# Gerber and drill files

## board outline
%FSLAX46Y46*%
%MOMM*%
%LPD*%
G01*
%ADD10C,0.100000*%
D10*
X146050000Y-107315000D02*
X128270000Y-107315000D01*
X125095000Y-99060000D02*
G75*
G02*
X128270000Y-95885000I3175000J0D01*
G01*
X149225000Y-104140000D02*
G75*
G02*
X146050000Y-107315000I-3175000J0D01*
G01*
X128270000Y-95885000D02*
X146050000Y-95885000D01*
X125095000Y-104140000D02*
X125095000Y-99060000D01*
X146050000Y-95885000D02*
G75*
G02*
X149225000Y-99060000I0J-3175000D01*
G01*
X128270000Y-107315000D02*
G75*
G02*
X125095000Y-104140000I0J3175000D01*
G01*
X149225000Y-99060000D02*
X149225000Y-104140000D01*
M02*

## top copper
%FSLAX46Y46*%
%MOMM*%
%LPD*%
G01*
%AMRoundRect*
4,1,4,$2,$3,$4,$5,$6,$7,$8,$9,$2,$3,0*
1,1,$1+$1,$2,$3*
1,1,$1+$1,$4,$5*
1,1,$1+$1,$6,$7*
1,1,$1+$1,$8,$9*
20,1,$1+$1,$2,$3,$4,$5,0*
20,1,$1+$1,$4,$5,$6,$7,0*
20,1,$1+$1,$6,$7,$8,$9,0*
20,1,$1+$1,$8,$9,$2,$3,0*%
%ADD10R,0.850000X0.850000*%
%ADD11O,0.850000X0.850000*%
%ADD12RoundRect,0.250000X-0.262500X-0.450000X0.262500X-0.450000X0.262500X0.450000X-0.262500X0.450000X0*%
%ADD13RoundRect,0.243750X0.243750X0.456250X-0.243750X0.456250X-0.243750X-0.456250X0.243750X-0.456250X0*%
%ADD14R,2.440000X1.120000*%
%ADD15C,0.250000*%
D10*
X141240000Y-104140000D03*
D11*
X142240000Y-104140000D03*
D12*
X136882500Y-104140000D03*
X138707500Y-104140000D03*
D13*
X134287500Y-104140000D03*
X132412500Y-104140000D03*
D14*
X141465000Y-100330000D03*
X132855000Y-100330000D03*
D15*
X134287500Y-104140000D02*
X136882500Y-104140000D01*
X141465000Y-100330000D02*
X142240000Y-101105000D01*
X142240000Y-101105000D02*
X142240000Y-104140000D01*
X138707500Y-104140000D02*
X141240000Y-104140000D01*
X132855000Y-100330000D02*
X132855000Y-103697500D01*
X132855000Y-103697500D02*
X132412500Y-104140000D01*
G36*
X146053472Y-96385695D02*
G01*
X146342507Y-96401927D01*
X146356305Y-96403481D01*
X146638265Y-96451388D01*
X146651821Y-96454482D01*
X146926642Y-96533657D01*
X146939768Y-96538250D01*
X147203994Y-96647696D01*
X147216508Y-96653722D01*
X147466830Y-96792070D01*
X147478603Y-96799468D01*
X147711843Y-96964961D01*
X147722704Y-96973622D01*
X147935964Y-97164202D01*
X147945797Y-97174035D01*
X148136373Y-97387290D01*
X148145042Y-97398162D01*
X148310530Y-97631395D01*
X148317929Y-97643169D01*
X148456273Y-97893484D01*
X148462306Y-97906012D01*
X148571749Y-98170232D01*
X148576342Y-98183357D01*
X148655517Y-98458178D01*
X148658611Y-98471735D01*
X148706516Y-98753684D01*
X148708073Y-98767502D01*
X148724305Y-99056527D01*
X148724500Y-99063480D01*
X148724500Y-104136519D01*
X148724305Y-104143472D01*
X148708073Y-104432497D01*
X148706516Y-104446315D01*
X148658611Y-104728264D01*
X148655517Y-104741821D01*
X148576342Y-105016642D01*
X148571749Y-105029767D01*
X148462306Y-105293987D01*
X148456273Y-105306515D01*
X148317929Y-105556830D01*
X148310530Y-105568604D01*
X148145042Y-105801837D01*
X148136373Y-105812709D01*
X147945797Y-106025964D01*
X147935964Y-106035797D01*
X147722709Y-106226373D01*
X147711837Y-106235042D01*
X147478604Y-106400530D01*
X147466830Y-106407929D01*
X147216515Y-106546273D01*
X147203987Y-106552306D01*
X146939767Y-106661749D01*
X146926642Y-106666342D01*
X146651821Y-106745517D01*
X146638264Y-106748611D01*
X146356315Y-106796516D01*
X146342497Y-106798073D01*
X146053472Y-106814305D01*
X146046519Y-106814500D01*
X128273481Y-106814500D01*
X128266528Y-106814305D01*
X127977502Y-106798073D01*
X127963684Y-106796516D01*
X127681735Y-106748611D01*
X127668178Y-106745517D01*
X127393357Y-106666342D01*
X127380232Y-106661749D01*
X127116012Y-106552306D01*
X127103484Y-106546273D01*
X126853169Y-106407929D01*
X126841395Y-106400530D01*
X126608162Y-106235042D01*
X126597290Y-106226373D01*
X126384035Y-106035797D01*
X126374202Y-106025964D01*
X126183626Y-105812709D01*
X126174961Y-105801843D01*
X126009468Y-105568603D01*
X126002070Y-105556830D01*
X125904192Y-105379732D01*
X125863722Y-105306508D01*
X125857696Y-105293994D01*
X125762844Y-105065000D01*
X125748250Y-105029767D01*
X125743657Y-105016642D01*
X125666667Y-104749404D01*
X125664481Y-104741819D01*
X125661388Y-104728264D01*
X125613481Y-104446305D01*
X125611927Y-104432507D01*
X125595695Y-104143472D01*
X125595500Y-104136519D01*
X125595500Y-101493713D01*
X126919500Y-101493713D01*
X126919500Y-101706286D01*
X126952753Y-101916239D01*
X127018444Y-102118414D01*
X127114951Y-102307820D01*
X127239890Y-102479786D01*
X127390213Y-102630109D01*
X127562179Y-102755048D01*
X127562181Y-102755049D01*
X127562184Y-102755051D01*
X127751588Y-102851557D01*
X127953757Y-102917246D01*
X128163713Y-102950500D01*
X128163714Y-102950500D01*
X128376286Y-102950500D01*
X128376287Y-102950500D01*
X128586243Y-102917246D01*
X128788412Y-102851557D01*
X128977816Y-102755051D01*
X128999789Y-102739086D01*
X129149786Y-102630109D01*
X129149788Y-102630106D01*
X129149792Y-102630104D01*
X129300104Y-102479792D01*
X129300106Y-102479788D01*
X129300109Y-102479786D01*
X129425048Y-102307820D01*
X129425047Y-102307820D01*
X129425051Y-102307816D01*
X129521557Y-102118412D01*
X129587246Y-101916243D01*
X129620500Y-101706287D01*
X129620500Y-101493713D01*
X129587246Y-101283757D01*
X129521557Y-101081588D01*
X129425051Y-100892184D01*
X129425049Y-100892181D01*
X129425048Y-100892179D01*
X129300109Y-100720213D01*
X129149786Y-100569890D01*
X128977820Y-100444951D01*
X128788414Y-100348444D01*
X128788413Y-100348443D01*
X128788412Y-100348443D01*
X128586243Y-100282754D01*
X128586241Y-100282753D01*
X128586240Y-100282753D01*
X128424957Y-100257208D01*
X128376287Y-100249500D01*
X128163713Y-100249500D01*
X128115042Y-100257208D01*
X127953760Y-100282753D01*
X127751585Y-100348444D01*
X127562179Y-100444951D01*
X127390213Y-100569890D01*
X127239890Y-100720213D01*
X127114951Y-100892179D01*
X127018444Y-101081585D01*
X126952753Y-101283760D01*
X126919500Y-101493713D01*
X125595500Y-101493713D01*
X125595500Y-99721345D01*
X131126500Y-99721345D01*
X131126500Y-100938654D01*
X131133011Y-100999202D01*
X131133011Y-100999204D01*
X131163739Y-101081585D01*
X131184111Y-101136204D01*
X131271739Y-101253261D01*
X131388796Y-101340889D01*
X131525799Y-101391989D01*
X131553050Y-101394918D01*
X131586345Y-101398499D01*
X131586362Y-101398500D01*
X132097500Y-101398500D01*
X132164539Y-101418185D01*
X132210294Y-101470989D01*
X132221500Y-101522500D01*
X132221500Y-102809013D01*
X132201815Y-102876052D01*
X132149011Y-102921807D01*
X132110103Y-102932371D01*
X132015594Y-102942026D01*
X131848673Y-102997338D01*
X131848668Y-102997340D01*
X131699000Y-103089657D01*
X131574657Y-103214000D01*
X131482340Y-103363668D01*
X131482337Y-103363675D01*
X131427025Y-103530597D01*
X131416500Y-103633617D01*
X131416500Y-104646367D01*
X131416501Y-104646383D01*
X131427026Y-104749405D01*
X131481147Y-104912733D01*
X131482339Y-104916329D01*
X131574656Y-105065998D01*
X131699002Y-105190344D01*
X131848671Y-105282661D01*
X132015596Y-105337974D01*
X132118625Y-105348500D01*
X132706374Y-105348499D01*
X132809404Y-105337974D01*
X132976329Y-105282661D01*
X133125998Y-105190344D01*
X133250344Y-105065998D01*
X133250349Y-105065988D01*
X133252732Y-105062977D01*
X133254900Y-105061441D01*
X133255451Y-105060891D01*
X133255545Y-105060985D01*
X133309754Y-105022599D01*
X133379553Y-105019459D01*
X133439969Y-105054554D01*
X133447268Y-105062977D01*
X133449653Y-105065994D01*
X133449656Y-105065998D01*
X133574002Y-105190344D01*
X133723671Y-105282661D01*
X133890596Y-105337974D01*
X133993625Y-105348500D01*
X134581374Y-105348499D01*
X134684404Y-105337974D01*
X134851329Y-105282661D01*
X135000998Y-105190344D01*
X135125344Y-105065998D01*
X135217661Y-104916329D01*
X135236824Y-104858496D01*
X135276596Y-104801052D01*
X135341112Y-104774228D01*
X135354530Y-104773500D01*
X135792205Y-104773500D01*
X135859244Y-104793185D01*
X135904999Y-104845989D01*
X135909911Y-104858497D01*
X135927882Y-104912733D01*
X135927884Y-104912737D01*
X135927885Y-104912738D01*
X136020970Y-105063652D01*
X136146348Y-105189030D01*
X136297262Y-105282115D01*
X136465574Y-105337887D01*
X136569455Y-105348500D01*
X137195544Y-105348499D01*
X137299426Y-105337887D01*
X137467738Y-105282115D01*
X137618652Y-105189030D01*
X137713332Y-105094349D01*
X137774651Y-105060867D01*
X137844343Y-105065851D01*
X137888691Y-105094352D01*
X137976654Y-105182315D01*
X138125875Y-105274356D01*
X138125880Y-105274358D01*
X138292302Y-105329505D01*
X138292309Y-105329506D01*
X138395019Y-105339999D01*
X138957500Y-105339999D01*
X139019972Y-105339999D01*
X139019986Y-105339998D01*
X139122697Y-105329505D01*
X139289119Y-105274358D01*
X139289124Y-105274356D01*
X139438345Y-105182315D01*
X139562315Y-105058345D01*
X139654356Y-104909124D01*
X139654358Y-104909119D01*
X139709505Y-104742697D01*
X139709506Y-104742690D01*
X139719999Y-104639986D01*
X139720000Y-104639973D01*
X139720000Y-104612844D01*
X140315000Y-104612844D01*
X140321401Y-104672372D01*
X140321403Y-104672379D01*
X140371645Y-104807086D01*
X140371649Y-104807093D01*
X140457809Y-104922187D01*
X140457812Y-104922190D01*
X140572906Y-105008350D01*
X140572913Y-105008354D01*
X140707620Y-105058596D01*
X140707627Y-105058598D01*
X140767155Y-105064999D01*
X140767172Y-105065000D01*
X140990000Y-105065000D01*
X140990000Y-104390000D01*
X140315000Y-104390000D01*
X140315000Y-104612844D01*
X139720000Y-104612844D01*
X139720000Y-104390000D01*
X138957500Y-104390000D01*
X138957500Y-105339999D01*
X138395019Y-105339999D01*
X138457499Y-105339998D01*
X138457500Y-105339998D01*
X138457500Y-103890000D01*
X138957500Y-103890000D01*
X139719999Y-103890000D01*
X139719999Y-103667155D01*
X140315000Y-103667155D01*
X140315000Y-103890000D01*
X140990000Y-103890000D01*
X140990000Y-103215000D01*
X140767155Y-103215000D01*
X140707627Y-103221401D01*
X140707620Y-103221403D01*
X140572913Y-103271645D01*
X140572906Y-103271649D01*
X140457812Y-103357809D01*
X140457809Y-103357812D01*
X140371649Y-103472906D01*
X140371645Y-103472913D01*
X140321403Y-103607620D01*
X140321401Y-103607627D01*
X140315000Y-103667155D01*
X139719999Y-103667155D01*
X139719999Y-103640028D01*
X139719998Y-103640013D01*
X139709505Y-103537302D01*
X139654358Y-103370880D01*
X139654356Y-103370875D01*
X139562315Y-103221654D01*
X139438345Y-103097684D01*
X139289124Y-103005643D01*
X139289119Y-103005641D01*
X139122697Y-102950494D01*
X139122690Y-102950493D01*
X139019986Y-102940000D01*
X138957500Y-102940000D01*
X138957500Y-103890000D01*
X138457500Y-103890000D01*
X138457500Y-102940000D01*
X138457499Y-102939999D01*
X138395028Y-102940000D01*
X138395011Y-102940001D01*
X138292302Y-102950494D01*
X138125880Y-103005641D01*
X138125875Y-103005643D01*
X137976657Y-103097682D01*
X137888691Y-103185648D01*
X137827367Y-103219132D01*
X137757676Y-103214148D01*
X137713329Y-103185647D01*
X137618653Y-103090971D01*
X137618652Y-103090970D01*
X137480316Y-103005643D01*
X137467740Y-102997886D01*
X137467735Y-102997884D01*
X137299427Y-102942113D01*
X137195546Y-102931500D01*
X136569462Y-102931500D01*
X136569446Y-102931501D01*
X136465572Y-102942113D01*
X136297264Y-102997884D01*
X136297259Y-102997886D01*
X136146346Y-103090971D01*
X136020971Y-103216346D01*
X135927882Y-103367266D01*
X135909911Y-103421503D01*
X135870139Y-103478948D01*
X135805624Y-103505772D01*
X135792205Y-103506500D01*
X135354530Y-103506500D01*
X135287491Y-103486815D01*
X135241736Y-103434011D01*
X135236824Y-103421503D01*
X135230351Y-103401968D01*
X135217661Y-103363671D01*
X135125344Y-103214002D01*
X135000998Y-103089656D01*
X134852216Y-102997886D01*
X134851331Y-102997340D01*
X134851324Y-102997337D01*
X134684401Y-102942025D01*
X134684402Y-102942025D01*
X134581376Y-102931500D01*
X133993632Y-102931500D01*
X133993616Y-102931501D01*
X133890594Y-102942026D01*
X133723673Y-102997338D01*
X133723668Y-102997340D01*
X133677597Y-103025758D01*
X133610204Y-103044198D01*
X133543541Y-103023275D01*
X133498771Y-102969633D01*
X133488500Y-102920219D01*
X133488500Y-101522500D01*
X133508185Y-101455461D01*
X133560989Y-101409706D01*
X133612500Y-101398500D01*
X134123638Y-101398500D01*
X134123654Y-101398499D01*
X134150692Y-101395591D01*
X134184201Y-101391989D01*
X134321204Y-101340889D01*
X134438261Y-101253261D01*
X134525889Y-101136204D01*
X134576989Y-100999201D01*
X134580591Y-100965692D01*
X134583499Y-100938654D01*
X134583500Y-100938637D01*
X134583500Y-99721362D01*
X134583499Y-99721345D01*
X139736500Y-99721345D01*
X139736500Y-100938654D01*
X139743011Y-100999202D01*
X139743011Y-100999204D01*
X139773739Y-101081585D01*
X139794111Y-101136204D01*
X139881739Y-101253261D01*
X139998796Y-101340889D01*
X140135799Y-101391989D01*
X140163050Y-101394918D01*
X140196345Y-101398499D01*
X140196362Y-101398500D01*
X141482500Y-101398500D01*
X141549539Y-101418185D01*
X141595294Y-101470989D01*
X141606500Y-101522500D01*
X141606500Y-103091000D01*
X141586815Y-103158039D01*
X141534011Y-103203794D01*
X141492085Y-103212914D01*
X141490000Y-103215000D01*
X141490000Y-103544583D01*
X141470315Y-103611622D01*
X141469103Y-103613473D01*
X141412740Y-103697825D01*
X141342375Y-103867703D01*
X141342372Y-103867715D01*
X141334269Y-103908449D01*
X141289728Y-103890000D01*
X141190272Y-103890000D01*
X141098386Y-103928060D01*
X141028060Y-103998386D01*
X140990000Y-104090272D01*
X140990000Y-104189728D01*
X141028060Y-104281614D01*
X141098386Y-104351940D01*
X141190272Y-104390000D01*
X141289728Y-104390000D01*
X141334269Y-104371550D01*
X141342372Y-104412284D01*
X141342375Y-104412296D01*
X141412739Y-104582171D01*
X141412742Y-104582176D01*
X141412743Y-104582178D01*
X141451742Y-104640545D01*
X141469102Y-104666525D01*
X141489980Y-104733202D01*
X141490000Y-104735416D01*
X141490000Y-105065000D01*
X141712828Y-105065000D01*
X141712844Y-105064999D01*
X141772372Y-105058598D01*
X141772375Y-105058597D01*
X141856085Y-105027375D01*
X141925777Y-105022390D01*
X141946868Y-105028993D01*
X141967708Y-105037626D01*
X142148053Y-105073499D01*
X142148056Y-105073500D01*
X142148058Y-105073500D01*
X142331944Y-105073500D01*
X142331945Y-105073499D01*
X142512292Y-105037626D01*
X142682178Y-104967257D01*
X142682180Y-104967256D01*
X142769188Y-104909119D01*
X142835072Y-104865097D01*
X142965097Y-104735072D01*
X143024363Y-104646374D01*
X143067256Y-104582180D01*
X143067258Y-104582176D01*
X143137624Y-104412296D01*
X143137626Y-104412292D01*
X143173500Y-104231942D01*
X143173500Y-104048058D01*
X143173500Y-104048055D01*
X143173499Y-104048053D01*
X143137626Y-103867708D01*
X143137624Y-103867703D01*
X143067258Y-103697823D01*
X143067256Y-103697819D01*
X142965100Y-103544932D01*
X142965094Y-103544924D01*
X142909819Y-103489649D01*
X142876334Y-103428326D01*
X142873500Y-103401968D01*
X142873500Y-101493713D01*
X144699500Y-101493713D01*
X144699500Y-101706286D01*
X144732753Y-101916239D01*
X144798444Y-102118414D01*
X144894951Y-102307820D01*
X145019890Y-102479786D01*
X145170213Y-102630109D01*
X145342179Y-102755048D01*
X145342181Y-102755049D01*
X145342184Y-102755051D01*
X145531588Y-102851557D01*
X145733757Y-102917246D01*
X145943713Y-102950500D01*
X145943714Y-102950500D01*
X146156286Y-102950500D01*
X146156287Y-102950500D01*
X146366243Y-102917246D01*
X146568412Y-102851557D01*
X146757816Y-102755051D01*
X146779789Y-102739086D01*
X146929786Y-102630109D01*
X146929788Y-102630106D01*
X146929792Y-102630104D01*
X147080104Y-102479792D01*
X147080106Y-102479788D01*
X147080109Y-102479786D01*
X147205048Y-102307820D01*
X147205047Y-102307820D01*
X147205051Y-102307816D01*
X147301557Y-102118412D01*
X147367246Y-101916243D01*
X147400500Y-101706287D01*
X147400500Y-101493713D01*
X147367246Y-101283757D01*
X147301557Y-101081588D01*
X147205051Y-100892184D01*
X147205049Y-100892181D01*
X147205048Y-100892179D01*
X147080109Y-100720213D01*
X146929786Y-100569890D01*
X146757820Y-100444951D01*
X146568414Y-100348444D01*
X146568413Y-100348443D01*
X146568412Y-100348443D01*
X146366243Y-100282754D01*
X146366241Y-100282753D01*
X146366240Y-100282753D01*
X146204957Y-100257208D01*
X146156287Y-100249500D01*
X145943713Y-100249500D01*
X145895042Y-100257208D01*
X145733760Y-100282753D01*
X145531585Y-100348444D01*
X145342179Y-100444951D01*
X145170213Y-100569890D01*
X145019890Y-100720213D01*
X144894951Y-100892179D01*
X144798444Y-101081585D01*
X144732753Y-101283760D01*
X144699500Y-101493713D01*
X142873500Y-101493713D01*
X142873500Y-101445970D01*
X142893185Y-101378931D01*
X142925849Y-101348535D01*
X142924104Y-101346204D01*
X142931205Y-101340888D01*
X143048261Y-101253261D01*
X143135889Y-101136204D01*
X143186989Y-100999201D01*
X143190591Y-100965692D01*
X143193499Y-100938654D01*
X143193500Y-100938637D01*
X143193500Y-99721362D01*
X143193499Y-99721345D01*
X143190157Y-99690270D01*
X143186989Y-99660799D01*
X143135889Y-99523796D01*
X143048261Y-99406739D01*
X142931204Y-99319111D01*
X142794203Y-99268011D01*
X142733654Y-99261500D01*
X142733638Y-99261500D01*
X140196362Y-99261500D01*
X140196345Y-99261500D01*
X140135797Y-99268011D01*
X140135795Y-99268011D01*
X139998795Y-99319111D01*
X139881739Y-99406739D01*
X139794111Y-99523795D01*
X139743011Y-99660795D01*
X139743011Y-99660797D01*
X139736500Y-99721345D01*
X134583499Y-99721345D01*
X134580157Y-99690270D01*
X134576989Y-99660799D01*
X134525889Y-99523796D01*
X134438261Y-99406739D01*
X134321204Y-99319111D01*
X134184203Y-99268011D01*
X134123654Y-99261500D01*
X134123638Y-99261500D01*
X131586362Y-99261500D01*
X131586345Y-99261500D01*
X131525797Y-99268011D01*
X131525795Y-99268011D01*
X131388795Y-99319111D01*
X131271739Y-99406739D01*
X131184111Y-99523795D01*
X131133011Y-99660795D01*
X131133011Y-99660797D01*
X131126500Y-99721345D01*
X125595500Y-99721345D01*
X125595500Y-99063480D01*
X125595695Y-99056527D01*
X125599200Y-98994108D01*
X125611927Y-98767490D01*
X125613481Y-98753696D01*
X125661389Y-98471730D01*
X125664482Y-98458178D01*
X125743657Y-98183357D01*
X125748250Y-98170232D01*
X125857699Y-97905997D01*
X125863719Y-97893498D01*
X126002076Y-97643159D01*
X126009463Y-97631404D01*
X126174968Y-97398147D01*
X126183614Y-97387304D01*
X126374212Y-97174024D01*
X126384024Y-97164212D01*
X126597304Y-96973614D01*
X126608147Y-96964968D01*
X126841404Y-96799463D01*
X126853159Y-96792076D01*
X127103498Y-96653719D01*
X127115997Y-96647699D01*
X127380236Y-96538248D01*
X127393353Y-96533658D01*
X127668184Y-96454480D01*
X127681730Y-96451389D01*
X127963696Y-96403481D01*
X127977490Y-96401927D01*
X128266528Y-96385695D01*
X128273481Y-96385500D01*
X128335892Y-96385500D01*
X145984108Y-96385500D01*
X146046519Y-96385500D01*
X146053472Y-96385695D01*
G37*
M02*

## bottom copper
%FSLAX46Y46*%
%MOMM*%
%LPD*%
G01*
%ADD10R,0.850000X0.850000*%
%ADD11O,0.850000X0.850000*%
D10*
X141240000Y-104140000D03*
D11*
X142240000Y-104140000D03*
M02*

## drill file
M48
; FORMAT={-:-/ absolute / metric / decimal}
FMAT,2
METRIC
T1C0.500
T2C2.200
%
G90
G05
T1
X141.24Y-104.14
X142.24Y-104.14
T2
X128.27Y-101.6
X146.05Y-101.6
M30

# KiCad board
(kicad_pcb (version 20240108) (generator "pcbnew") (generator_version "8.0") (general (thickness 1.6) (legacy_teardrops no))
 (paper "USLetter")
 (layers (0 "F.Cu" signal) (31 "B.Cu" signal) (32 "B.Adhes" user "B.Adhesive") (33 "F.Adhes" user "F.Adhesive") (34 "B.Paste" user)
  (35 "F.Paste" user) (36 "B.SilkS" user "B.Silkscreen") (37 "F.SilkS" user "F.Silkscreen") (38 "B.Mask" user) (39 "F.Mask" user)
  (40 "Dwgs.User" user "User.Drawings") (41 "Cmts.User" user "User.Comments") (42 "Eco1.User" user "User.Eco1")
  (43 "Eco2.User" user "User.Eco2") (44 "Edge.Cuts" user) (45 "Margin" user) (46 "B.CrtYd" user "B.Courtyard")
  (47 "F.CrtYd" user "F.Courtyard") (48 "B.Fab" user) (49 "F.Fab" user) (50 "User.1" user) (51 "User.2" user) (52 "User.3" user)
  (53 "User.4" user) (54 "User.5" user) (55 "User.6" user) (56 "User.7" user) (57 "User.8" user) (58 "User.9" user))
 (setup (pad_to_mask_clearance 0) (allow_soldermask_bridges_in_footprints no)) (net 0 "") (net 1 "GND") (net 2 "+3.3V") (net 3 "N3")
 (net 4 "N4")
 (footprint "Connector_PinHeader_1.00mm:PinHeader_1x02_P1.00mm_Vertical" (layer "F.Cu") (at 141.24 104.14 90)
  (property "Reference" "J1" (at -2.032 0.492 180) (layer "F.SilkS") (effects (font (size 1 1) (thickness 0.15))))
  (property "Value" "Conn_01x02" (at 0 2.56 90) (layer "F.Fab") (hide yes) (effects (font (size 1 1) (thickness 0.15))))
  (pad "1" thru_hole rect (at 0 0 90) (size 0.85 0.85) (drill 0.5) (layers "*.Cu" "*.Mask") (remove_unused_layers no) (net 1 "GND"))
  (pad "2" thru_hole oval (at 0 1 90) (size 0.85 0.85) (drill 0.5) (layers "*.Cu" "*.Mask") (remove_unused_layers no) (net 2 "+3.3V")))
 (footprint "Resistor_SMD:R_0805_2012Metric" (layer "F.Cu") (at 137.795 104.14)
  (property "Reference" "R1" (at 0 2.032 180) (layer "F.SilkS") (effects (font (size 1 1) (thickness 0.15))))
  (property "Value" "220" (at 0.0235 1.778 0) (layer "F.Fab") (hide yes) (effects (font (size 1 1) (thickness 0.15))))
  (pad "1" smd roundrect (at -0.9125 0) (size 1.025 1.4) (layers "F.Cu" "F.Paste" "F.Mask") (roundrect_rratio 0.243902) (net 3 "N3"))
  (pad "2" smd roundrect (at 0.9125 0) (size 1.025 1.4) (layers "F.Cu" "F.Paste" "F.Mask") (roundrect_rratio 0.243902) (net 1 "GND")))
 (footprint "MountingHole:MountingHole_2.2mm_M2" (layer "F.Cu") (at 146.05 101.6 90)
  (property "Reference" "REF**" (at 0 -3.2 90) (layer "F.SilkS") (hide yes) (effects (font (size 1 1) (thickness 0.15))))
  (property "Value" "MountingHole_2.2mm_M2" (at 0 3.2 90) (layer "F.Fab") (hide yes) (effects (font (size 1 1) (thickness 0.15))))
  (pad "" np_thru_hole circle (at 0 0 90) (size 2.2 2.2) (drill 2.2) (layers "*.Cu" "*.Mask")))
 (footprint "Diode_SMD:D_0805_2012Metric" (layer "F.Cu") (at 133.35 104.14 180)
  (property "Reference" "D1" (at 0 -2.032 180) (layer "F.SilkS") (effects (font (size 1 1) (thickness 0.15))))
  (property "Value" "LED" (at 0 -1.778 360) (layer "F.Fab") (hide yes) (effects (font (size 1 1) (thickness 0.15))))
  (pad "1" smd roundrect (at -0.9375 0 180) (size 0.975 1.4) (layers "F.Cu" "F.Paste" "F.Mask") (roundrect_rratio 0.25) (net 3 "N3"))
  (pad "2" smd roundrect (at 0.9375 0 180) (size 0.975 1.4) (layers "F.Cu" "F.Paste" "F.Mask") (roundrect_rratio 0.25) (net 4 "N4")))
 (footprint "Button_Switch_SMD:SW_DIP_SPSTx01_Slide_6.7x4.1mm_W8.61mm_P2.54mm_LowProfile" (layer "F.Cu") (at 137.16 100.33 180)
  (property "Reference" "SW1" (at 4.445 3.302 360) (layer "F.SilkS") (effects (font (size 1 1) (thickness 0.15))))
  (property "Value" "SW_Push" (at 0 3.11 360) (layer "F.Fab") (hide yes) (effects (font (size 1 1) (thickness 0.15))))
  (pad "1" smd rect (at -4.305 0 180) (size 2.44 1.12) (layers "F.Cu" "F.Paste" "F.Mask") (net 2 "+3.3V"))
  (pad "2" smd rect (at 4.305 0 180) (size 2.44 1.12) (layers "F.Cu" "F.Paste" "F.Mask") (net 4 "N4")))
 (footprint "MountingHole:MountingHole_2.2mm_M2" (layer "F.Cu") (at 128.27 101.6 90)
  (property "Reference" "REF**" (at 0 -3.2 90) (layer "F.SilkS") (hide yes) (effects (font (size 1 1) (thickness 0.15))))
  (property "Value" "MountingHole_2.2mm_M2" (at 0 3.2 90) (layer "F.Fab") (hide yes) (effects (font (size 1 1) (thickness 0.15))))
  (pad "" np_thru_hole circle (at 0 0 90) (size 2.2 2.2) (drill 2.2) (layers "*.Cu" "*.Mask")))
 (gr_line (start 146.05 107.315) (end 128.27 107.315) (stroke (width 0.1) (type default)) (layer "Edge.Cuts"))
 (gr_arc (start 125.095 99.06) (mid 126.024936 96.814936) (end 128.27 95.885) (stroke (width 0.1) (type default)) (layer "Edge.Cuts"))
 (gr_arc (start 149.225 104.14) (mid 148.295064 106.385064) (end 146.05 107.315) (stroke (width 0.1) (type default)) (layer "Edge.Cuts"))
 (gr_line (start 128.27 95.885) (end 146.05 95.885) (stroke (width 0.1) (type default)) (layer "Edge.Cuts"))
 (gr_line (start 125.095 104.14) (end 125.095 99.06) (stroke (width 0.1) (type default)) (layer "Edge.Cuts"))
 (gr_arc (start 146.05 95.885) (mid 148.295064 96.814936) (end 149.225 99.06) (stroke (width 0.1) (type default)) (layer "Edge.Cuts"))
 (gr_arc (start 128.27 107.315) (mid 126.024936 106.385064) (end 125.095 104.14) (stroke (width 0.1) (type default)) (layer "Edge.Cuts"))
 (gr_line (start 149.225 99.06) (end 149.225 104.14) (stroke (width 0.1) (type default)) (layer "Edge.Cuts"))
 (segment (start 134.2875 104.14) (end 136.8825 104.14) (width 0.25) (layer "F.Cu") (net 3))
 (segment (start 141.465 100.33) (end 142.24 101.105) (width 0.25) (layer "F.Cu") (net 2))
 (segment (start 142.24 101.105) (end 142.24 104.14) (width 0.25) (layer "F.Cu") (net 2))
 (segment (start 138.7075 104.14) (end 141.24 104.14) (width 0.25) (layer "F.Cu") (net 1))
 (segment (start 132.855 100.33) (end 132.855 103.6975) (width 0.25) (layer "F.Cu") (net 4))
 (segment (start 132.855 103.6975) (end 132.4125 104.14) (width 0.25) (layer "F.Cu") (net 4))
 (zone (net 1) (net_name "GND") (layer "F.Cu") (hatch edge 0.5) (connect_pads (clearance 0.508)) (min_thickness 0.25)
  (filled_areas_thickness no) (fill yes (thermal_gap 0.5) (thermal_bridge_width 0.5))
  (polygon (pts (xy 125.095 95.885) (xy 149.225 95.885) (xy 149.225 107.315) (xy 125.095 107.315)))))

